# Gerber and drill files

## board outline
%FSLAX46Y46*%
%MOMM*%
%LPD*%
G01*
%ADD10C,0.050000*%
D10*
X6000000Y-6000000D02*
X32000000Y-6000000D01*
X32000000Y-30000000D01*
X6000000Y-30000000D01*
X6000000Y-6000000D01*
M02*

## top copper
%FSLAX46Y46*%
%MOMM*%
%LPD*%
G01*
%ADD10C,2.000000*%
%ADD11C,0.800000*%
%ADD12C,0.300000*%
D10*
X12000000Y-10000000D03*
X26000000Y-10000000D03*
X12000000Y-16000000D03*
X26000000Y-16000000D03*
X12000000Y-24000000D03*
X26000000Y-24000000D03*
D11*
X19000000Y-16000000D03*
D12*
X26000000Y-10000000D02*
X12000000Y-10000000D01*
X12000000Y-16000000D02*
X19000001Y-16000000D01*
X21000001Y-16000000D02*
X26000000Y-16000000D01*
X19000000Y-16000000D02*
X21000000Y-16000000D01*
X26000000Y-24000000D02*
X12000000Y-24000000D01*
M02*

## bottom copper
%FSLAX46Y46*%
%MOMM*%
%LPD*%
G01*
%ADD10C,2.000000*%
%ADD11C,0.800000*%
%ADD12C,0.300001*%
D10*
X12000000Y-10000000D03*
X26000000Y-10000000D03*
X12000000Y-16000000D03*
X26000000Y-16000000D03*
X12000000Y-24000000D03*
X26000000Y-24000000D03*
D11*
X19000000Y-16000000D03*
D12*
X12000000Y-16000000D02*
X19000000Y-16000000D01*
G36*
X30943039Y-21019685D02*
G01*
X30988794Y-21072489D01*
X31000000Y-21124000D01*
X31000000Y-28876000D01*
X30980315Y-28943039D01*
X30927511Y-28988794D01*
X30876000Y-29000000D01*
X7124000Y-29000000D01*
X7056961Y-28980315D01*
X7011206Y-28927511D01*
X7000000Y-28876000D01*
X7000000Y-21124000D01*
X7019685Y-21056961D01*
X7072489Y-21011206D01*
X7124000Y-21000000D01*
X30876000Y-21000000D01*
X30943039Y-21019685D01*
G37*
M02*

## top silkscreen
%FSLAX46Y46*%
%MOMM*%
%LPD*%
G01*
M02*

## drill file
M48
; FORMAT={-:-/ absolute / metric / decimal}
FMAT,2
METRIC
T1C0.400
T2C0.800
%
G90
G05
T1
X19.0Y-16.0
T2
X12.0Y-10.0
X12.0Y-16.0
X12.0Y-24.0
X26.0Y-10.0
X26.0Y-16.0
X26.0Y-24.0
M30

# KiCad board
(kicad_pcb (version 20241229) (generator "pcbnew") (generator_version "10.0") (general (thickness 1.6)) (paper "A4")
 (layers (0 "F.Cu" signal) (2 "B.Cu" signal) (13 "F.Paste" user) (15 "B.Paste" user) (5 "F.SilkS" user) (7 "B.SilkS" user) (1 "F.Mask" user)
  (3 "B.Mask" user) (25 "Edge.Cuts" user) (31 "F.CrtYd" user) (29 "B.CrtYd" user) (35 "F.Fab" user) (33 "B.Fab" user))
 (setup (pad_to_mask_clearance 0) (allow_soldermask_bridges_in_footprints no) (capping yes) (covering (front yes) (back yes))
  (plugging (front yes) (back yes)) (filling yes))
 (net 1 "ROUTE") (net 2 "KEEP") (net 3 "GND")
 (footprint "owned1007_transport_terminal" (layer "F.Cu") (at 12 10)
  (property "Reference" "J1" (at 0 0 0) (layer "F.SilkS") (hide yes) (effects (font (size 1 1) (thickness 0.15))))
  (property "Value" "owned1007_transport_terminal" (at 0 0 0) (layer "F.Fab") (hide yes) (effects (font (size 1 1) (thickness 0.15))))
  (pad "1" thru_hole circle (at 0 0) (size 2 2) (drill 0.8) (layers "*.Cu" "*.Mask") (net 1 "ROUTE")))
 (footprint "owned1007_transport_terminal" (layer "F.Cu") (at 26 10)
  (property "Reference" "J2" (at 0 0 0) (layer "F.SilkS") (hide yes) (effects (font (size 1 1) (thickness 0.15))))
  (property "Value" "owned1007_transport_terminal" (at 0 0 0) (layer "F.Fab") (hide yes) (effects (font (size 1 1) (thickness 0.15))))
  (pad "1" thru_hole circle (at 0 0) (size 2 2) (drill 0.8) (layers "*.Cu" "*.Mask") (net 1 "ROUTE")))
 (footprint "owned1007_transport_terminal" (layer "F.Cu") (at 12 16)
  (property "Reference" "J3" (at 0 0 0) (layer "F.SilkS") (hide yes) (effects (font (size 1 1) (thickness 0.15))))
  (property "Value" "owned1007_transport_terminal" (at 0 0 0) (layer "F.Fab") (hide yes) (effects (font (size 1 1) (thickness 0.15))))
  (pad "1" thru_hole circle (at 0 0) (size 2 2) (drill 0.8) (layers "*.Cu" "*.Mask") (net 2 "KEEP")))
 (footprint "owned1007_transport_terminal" (layer "F.Cu") (at 26 16)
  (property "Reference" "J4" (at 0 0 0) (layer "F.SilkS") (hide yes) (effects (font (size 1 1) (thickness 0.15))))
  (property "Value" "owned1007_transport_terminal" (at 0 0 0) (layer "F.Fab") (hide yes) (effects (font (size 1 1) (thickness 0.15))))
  (pad "1" thru_hole circle (at 0 0) (size 2 2) (drill 0.8) (layers "*.Cu" "*.Mask") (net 2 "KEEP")))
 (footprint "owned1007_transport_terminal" (layer "F.Cu") (at 12 24)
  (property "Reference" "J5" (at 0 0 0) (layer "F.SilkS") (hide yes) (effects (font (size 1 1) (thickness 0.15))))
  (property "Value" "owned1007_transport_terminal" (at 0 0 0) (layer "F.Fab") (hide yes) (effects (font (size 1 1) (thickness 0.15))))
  (pad "1" thru_hole circle (at 0 0) (size 2 2) (drill 0.8) (layers "*.Cu" "*.Mask") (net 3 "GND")))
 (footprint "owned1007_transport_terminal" (layer "F.Cu") (at 26 24)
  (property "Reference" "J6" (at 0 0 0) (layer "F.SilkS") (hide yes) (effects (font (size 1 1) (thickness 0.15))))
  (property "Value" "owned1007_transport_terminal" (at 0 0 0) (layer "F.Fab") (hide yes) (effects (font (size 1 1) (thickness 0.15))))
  (pad "1" thru_hole circle (at 0 0) (size 2 2) (drill 0.8) (layers "*.Cu" "*.Mask") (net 3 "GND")))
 (gr_rect (start 6 6) (end 32 30) (stroke (width 0.05) (type default)) (fill none) (layer "Edge.Cuts"))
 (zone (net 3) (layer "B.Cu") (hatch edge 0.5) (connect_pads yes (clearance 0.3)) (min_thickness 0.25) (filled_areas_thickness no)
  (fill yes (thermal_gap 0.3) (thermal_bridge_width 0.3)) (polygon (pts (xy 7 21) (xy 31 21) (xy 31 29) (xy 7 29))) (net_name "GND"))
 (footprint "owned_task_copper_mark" (layer "F.Cu") (at 10 28)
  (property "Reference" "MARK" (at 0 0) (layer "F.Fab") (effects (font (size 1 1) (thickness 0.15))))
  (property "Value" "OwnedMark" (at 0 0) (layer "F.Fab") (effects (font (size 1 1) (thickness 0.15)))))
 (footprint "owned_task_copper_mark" (layer "F.Cu") (at 13 28)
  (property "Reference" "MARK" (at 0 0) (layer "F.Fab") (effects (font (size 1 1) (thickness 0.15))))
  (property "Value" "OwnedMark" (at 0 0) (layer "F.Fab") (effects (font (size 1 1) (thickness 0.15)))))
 (segment (start 26 10) (end 12 10) (width 0.3) (layer "F.Cu") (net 1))
 (segment (start 12 16) (end 19.000001 16) (width 0.3) (layer "F.Cu") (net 2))
 (segment (start 21.000001 16) (end 26 16) (width 0.3) (layer "F.Cu") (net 2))
 (segment (start 19 16) (end 21 16) (width 0.3) (layer "F.Cu") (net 2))
 (via (at 19 16) (size 0.8) (drill 0.4) (layers "F.Cu" "B.Cu") (free yes) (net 2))
 (segment (start 12 16) (end 19 16) (width 0.300001) (layer "B.Cu") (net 2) (locked yes))
 (segment (start 26 24) (end 12 24) (width 0.3) (layer "F.Cu") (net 3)))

